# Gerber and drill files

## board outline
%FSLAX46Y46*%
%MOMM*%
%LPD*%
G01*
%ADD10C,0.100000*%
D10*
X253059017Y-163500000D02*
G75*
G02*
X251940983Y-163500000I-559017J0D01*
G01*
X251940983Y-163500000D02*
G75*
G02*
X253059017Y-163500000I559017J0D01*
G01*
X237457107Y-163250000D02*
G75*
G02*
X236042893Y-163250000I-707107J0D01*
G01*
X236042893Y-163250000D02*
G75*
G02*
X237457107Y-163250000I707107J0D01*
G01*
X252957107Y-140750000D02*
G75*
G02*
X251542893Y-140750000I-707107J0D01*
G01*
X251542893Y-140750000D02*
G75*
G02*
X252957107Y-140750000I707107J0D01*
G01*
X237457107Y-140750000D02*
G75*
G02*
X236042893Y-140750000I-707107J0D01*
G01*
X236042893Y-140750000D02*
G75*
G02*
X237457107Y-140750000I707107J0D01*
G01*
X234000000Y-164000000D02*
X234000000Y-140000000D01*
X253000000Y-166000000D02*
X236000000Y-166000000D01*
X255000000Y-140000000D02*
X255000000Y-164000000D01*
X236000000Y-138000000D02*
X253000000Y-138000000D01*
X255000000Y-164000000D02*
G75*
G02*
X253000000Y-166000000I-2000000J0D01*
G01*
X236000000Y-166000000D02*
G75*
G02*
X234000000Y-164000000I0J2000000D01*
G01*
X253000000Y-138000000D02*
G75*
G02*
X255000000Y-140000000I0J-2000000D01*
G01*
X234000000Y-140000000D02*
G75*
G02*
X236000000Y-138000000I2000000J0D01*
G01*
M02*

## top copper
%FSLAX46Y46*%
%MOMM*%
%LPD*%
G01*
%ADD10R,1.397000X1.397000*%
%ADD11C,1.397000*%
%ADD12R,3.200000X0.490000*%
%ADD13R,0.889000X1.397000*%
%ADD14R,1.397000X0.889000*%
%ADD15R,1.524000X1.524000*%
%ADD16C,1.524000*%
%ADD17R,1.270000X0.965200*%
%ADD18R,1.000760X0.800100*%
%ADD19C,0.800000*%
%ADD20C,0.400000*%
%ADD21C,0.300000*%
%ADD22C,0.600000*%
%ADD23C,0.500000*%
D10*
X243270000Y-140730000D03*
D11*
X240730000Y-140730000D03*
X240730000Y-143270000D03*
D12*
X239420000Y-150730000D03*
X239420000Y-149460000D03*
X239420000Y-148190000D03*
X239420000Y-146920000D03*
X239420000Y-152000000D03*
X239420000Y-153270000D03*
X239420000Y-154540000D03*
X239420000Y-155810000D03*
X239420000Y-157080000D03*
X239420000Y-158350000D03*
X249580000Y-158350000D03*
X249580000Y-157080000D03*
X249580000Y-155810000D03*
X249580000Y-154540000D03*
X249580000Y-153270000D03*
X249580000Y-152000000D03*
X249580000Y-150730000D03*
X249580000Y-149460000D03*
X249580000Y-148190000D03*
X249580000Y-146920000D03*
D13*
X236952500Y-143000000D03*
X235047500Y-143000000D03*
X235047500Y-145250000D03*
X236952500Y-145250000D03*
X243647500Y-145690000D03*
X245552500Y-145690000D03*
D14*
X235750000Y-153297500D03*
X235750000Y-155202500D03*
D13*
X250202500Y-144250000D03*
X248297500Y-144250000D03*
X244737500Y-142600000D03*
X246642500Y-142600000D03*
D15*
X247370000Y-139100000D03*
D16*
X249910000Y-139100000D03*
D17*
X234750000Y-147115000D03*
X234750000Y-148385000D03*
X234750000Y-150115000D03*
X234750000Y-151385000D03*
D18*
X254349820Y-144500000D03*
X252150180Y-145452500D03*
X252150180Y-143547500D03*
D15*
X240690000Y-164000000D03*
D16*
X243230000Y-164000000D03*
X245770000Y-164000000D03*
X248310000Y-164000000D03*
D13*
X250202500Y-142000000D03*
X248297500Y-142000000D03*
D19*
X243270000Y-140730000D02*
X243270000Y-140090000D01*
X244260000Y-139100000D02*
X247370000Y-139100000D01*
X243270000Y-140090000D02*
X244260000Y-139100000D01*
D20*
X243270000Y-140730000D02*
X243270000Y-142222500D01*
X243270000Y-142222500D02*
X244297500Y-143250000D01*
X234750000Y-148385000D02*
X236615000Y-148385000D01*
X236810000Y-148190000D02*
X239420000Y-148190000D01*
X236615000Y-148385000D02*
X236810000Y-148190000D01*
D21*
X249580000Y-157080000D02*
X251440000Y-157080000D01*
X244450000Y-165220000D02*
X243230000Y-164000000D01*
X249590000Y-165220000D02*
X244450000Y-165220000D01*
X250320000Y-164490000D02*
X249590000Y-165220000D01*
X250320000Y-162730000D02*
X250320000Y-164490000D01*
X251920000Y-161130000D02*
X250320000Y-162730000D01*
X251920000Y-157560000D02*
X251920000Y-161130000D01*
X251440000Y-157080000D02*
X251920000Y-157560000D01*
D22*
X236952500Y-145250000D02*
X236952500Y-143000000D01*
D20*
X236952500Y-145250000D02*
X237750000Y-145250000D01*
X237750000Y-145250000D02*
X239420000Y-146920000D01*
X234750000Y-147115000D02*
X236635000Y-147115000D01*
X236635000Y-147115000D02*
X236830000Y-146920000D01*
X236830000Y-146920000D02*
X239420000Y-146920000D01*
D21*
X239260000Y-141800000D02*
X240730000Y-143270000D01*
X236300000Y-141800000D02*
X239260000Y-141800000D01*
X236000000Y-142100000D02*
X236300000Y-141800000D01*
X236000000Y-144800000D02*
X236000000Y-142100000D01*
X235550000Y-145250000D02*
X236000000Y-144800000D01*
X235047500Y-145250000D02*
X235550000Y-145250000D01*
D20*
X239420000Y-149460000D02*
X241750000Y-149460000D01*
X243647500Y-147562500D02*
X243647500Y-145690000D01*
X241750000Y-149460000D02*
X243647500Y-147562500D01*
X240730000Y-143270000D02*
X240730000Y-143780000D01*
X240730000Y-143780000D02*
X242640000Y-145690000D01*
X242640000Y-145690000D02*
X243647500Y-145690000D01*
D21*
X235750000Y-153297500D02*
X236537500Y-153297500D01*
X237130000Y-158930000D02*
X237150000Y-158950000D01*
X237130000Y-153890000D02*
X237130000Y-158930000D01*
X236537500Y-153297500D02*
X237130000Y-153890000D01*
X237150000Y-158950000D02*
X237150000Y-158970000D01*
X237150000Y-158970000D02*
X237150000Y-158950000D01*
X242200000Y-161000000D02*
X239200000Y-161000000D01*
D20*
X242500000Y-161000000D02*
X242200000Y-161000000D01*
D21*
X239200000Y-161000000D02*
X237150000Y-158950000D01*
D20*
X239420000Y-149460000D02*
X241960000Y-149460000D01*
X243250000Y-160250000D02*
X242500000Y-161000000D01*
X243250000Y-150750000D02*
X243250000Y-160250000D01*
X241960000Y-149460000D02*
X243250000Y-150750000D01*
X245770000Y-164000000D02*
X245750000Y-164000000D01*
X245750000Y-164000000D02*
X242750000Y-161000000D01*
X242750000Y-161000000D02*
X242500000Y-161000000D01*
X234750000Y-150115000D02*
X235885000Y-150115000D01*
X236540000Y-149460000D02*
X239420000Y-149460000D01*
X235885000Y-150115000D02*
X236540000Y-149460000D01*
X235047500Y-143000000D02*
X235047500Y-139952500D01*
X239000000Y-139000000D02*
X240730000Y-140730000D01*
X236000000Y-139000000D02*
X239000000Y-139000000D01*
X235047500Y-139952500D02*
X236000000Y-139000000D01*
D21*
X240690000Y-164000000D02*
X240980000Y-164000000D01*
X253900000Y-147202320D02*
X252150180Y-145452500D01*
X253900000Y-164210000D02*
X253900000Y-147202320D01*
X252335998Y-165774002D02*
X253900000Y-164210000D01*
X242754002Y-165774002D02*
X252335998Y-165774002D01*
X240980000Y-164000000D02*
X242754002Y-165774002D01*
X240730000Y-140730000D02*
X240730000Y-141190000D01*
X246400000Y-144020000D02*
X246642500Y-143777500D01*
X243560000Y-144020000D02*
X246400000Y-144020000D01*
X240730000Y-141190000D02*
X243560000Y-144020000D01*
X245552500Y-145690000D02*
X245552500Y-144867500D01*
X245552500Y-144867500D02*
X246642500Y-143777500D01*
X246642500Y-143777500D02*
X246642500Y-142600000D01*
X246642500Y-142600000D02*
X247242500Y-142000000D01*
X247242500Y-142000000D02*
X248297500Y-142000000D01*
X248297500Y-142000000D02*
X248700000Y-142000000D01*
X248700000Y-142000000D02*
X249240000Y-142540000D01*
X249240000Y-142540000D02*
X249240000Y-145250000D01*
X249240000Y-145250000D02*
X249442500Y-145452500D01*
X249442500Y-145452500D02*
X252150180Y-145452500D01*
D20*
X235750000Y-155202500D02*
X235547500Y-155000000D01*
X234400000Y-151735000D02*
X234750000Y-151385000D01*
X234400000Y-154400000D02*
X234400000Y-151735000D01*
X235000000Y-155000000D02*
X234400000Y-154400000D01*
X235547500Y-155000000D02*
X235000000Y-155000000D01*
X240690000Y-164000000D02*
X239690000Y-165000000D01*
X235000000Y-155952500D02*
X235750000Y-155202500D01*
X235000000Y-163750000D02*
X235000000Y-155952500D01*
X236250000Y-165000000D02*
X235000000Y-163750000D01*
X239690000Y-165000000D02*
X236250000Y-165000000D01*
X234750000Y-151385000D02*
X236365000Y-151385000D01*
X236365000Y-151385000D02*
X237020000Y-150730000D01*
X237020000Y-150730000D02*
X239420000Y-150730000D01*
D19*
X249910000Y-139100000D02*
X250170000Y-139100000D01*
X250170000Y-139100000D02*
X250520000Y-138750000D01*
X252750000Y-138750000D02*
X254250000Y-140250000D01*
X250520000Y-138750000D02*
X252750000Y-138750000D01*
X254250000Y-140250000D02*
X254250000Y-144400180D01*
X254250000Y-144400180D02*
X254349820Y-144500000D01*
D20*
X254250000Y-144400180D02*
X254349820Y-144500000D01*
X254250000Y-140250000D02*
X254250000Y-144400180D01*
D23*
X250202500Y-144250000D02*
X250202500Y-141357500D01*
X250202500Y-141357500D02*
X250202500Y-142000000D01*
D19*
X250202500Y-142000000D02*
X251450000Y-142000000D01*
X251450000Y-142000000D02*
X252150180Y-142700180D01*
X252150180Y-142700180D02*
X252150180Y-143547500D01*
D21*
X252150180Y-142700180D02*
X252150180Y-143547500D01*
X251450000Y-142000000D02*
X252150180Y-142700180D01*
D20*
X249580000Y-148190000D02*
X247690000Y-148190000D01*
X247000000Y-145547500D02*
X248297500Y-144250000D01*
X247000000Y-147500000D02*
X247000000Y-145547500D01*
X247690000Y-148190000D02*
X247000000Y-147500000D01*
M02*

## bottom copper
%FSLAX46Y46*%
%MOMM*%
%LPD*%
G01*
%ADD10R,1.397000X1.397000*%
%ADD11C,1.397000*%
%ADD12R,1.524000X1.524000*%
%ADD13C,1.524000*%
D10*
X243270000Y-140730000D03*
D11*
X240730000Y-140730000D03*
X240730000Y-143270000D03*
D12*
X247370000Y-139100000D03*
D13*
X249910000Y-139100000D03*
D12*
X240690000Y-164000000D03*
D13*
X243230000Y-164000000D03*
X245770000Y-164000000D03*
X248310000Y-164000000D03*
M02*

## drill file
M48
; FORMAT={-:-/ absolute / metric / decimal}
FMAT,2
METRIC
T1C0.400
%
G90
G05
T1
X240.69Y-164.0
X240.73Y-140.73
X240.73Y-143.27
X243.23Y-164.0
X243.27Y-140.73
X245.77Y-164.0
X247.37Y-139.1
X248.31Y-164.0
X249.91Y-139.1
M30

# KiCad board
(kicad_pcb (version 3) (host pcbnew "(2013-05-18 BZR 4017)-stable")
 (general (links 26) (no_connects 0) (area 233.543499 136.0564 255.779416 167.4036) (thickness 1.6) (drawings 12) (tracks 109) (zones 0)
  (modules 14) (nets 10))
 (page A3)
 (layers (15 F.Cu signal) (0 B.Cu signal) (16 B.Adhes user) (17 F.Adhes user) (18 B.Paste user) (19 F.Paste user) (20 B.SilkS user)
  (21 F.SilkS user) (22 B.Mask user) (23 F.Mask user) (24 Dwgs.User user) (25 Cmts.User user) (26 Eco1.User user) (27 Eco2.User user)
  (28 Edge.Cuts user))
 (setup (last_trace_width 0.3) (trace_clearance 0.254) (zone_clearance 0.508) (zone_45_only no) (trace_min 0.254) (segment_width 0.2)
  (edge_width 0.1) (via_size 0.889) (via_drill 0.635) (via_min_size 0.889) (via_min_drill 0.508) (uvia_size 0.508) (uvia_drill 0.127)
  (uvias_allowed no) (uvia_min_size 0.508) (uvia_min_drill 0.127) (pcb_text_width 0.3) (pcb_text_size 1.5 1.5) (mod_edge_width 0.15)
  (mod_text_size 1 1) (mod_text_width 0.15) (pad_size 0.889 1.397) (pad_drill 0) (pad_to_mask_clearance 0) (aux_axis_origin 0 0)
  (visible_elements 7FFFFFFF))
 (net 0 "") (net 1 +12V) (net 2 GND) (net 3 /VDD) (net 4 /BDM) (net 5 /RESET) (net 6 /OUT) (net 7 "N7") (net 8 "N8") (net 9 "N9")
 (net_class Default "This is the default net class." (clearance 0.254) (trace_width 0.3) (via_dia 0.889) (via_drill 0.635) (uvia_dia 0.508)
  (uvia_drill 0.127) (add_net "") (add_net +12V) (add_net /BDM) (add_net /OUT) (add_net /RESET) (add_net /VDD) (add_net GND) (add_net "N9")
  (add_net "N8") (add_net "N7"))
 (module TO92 (layer F.Cu) (at 242 142)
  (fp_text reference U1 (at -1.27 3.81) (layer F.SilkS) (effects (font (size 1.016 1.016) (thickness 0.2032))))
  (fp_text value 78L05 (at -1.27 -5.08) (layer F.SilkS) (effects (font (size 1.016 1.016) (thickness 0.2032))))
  (pad 1 thru_hole rect (at 1.27 -1.27) (size 1.397 1.397) (drill 0.4) (layers *.Cu *.Mask F.SilkS) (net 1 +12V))
  (pad 2 thru_hole circle (at -1.27 -1.27) (size 1.397 1.397) (drill 0.4) (layers *.Cu *.Mask F.SilkS) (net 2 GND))
  (pad 3 thru_hole circle (at -1.27 1.27) (size 1.397 1.397) (drill 0.4) (layers *.Cu *.Mask F.SilkS) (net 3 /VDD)))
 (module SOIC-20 (layer F.Cu) (at 244.5 152)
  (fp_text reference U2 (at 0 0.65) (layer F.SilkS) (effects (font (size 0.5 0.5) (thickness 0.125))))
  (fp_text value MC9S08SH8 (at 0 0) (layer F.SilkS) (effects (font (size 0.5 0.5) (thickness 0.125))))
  (pad 4 smd rect (at -5.08 -1.27) (size 3.2 0.49) (layers F.Cu F.Paste F.Mask) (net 2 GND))
  (pad 3 smd rect (at -5.08 -2.54) (size 3.2 0.49) (layers F.Cu F.Paste F.Mask) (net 3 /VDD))
  (pad 2 smd rect (at -5.08 -3.81) (size 3.2 0.49) (layers F.Cu F.Paste F.Mask) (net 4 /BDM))
  (pad 1 smd rect (at -5.08 -5.08) (size 3.2 0.49) (layers F.Cu F.Paste F.Mask) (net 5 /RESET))
  (pad 5 smd rect (at -5.08 0) (size 3.2 0.49) (layers F.Cu F.Paste F.Mask))
  (pad 6 smd rect (at -5.08 1.27) (size 3.2 0.49) (layers F.Cu F.Paste F.Mask))
  (pad 7 smd rect (at -5.08 2.54) (size 3.2 0.49) (layers F.Cu F.Paste F.Mask))
  (pad 8 smd rect (at -5.08 3.81) (size 3.2 0.49) (layers F.Cu F.Paste F.Mask))
  (pad 9 smd rect (at -5.08 5.08) (size 3.2 0.49) (layers F.Cu F.Paste F.Mask))
  (pad 10 smd rect (at -5.08 6.35) (size 3.2 0.49) (layers F.Cu F.Paste F.Mask))
  (pad 11 smd rect (at 5.08 6.35) (size 3.2 0.49) (layers F.Cu F.Paste F.Mask))
  (pad 12 smd rect (at 5.08 5.08) (size 3.2 0.49) (layers F.Cu F.Paste F.Mask) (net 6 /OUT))
  (pad 13 smd rect (at 5.08 3.81) (size 3.2 0.49) (layers F.Cu F.Paste F.Mask))
  (pad 14 smd rect (at 5.08 2.54) (size 3.2 0.49) (layers F.Cu F.Paste F.Mask))
  (pad 15 smd rect (at 5.08 1.27) (size 3.2 0.49) (layers F.Cu F.Paste F.Mask))
  (pad 16 smd rect (at 5.08 0) (size 3.2 0.49) (layers F.Cu F.Paste F.Mask))
  (pad 17 smd rect (at 5.08 -1.27) (size 3.2 0.49) (layers F.Cu F.Paste F.Mask))
  (pad 18 smd rect (at 5.08 -2.54) (size 3.2 0.49) (layers F.Cu F.Paste F.Mask))
  (pad 19 smd rect (at 5.08 -3.81) (size 3.2 0.49) (layers F.Cu F.Paste F.Mask) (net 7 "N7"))
  (pad 20 smd rect (at 5.08 -5.08) (size 3.2 0.49) (layers F.Cu F.Paste F.Mask)))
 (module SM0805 (layer F.Cu) (at 236 143 180)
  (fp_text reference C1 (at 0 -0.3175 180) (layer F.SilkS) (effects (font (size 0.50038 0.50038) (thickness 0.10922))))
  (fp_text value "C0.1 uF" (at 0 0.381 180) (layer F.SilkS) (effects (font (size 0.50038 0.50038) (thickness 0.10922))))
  (pad 1 smd rect (at -0.9525 0 180) (size 0.889 1.397) (layers F.Cu F.Paste F.Mask) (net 5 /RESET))
  (pad 2 smd rect (at 0.9525 0 180) (size 0.889 1.397) (layers F.Cu F.Paste F.Mask) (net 2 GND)))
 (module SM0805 (layer F.Cu) (at 236 145.25)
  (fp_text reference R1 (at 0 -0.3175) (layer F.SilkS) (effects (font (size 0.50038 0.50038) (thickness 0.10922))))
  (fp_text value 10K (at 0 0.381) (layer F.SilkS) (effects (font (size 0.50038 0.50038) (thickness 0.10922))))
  (pad 1 smd rect (at -0.9525 0) (size 0.889 1.397) (layers F.Cu F.Paste F.Mask) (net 3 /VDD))
  (pad 2 smd rect (at 0.9525 0) (size 0.889 1.397) (layers F.Cu F.Paste F.Mask) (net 5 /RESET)))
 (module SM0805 (layer F.Cu) (at 244.6 145.69)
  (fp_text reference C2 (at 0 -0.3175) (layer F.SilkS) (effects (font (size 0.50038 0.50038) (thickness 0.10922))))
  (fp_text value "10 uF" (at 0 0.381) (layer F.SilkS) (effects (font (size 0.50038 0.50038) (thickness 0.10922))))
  (pad 1 smd rect (at -0.9525 0) (size 0.889 1.397) (layers F.Cu F.Paste F.Mask) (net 3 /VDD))
  (pad 2 smd rect (at 0.9525 0) (size 0.889 1.397) (layers F.Cu F.Paste F.Mask) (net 2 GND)))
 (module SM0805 (layer F.Cu) (at 235.75 154.25 270)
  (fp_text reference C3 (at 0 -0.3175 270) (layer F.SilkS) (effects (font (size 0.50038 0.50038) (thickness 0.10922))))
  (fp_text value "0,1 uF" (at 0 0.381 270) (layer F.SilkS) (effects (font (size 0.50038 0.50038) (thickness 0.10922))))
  (pad 1 smd rect (at -0.9525 0 270) (size 0.889 1.397) (layers F.Cu F.Paste F.Mask) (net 3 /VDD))
  (pad 2 smd rect (at 0.9525 0 270) (size 0.889 1.397) (layers F.Cu F.Paste F.Mask) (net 2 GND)))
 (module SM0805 (layer F.Cu) (at 249.25 144.25 180)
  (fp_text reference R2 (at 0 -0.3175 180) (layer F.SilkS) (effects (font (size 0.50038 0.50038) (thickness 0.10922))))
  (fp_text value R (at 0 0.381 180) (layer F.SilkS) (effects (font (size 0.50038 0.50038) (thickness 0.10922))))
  (pad 1 smd rect (at -0.9525 0 180) (size 0.889 1.397) (layers F.Cu F.Paste F.Mask) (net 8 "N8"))
  (pad 2 smd rect (at 0.9525 0 180) (size 0.889 1.397) (layers F.Cu F.Paste F.Mask) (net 7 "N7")))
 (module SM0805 (layer F.Cu) (at 245.69 142.6)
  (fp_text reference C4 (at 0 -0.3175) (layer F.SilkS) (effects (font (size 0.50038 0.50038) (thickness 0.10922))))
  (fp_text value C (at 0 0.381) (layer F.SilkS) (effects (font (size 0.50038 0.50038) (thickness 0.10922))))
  (pad 1 smd rect (at -0.9525 0) (size 0.889 1.397) (layers F.Cu F.Paste F.Mask) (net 1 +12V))
  (pad 2 smd rect (at 0.9525 0) (size 0.889 1.397) (layers F.Cu F.Paste F.Mask) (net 2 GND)))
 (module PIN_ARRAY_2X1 (layer F.Cu) (at 248.64 139.1)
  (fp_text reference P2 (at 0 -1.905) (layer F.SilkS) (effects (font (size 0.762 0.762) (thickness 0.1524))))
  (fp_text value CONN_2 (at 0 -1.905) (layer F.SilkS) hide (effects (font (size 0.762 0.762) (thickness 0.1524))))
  (pad 1 thru_hole rect (at -1.27 0) (size 1.524 1.524) (drill 0.4) (layers *.Cu *.Mask F.SilkS) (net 1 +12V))
  (pad 2 thru_hole circle (at 1.27 0) (size 1.524 1.524) (drill 0.4) (layers *.Cu *.Mask F.SilkS) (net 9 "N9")))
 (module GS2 (layer F.Cu) (at 234.75 147.75)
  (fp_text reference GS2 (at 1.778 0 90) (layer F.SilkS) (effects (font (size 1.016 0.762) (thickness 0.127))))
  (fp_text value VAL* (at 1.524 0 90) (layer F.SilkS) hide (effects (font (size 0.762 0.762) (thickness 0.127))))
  (pad 1 smd rect (at 0 -0.635) (size 1.27 0.9652) (layers F.Cu F.Paste F.Mask) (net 5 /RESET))
  (pad 2 smd rect (at 0 0.635) (size 1.27 0.9652) (layers F.Cu F.Paste F.Mask) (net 4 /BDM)))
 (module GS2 (layer F.Cu) (at 234.75 150.75)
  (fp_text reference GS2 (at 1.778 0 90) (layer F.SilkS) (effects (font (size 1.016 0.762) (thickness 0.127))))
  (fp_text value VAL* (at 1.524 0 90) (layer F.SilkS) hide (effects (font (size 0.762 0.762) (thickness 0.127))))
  (pad 1 smd rect (at 0 -0.635) (size 1.27 0.9652) (layers F.Cu F.Paste F.Mask) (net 3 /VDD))
  (pad 2 smd rect (at 0 0.635) (size 1.27 0.9652) (layers F.Cu F.Paste F.Mask) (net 2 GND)))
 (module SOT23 (layer F.Cu) (at 253.25 144.5 270)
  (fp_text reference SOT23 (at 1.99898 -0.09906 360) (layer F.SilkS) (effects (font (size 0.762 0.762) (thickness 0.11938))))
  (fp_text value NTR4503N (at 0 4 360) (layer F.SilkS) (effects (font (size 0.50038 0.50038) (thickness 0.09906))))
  (pad 3 smd rect (at 0 -1.09982 270) (size 0.8001 1.00076) (layers F.Cu F.Paste F.Mask) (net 9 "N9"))
  (pad 2 smd rect (at 0.9525 1.09982 270) (size 0.8001 1.00076) (layers F.Cu F.Paste F.Mask) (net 2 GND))
  (pad 1 smd rect (at -0.9525 1.09982 270) (size 0.8001 1.00076) (layers F.Cu F.Paste F.Mask) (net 8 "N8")))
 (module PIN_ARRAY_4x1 (layer F.Cu) (at 244.5 164)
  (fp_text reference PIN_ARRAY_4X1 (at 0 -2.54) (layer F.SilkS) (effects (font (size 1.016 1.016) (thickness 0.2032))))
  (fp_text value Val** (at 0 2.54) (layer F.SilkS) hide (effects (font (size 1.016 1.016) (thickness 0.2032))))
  (pad 1 thru_hole rect (at -3.81 0) (size 1.524 1.524) (drill 0.4) (layers *.Cu *.Mask F.SilkS) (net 2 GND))
  (pad 2 thru_hole circle (at -1.27 0) (size 1.524 1.524) (drill 0.4) (layers *.Cu *.Mask F.SilkS) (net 6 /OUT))
  (pad 3 thru_hole circle (at 1.27 0) (size 1.524 1.524) (drill 0.4) (layers *.Cu *.Mask F.SilkS) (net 3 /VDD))
  (pad 4 thru_hole circle (at 3.81 0) (size 1.524 1.524) (drill 0.4) (layers *.Cu *.Mask F.SilkS)))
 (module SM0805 (layer F.Cu) (at 249.25 142 180)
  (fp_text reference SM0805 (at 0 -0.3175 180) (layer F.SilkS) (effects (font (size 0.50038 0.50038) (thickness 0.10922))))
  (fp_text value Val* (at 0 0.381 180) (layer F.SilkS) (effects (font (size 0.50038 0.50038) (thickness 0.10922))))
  (pad 1 smd rect (at -0.9525 0 180) (size 0.889 1.397) (layers F.Cu F.Paste F.Mask) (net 8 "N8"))
  (pad 2 smd rect (at 0.9525 0 180) (size 0.889 1.397) (layers F.Cu F.Paste F.Mask) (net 2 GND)))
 (gr_circle (center 252.5 163.5) (end 253 163.75) (layer Edge.Cuts) (width 0.1))
 (gr_circle (center 236.75 163.25) (end 237.25 163.75) (layer Edge.Cuts) (width 0.1))
 (gr_circle (center 252.25 140.75) (end 252.75 140.25) (layer Edge.Cuts) (width 0.1))
 (gr_circle (center 236.75 140.75) (end 236.25 140.25) (layer Edge.Cuts) (width 0.1))
 (gr_line (start 234 164) (end 234 140) (angle 90) (layer Edge.Cuts) (width 0.1))
 (gr_line (start 253 166) (end 236 166) (angle 90) (layer Edge.Cuts) (width 0.1))
 (gr_line (start 255 140) (end 255 164) (angle 90) (layer Edge.Cuts) (width 0.1))
 (gr_line (start 236 138) (end 253 138) (angle 90) (layer Edge.Cuts) (width 0.1))
 (gr_arc (start 253 164) (end 255 164) (angle 90) (layer Edge.Cuts) (width 0.1))
 (gr_arc (start 236 164) (end 236 166) (angle 90) (layer Edge.Cuts) (width 0.1))
 (gr_arc (start 253 140) (end 253 138) (angle 90) (layer Edge.Cuts) (width 0.1))
 (gr_arc (start 236 140) (end 234 140) (angle 90) (layer Edge.Cuts) (width 0.1))
 (segment (start 243.27 140.73) (end 243.27 140.09) (width 0.8) (layer F.Cu) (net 1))
 (segment (start 244.26 139.1) (end 247.37 139.1) (width 0.8) (layer F.Cu) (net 1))
 (segment (start 243.27 140.09) (end 244.26 139.1) (width 0.8) (layer F.Cu) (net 1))
 (segment (start 243.27 140.73) (end 243.27 142.2225) (width 0.4) (layer F.Cu) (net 1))
 (segment (start 243.27 142.2225) (end 244.2975 143.25) (width 0.4) (layer F.Cu) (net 1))
 (segment (start 234.75 148.385) (end 236.615 148.385) (width 0.4) (layer F.Cu) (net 4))
 (segment (start 236.81 148.19) (end 239.42 148.19) (width 0.4) (layer F.Cu) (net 4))
 (segment (start 236.615 148.385) (end 236.81 148.19) (width 0.4) (layer F.Cu) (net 4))
 (segment (start 249.58 157.08) (end 251.44 157.08) (width 0.3) (layer F.Cu) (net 6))
 (segment (start 244.45 165.22) (end 243.23 164) (width 0.3) (layer F.Cu) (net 6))
 (segment (start 249.59 165.22) (end 244.45 165.22) (width 0.3) (layer F.Cu) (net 6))
 (segment (start 250.32 164.49) (end 249.59 165.22) (width 0.3) (layer F.Cu) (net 6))
 (segment (start 250.32 162.73) (end 250.32 164.49) (width 0.3) (layer F.Cu) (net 6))
 (segment (start 251.92 161.13) (end 250.32 162.73) (width 0.3) (layer F.Cu) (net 6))
 (segment (start 251.92 157.56) (end 251.92 161.13) (width 0.3) (layer F.Cu) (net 6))
 (segment (start 251.44 157.08) (end 251.92 157.56) (width 0.3) (layer F.Cu) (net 6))
 (segment (start 236.9525 145.25) (end 236.9525 143) (width 0.6) (layer F.Cu) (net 5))
 (segment (start 236.9525 145.25) (end 237.75 145.25) (width 0.4) (layer F.Cu) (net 5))
 (segment (start 237.75 145.25) (end 239.42 146.92) (width 0.4) (layer F.Cu) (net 5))
 (segment (start 234.75 147.115) (end 236.635 147.115) (width 0.4) (layer F.Cu) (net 5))
 (segment (start 236.635 147.115) (end 236.83 146.92) (width 0.4) (layer F.Cu) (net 5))
 (segment (start 236.83 146.92) (end 239.42 146.92) (width 0.4) (layer F.Cu) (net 5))
 (segment (start 239.26 141.8) (end 240.73 143.27) (width 0.3) (layer F.Cu) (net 3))
 (segment (start 236.3 141.8) (end 239.26 141.8) (width 0.3) (layer F.Cu) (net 3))
 (segment (start 236 142.1) (end 236.3 141.8) (width 0.3) (layer F.Cu) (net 3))
 (segment (start 236 144.8) (end 236 142.1) (width 0.3) (layer F.Cu) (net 3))
 (segment (start 235.55 145.25) (end 236 144.8) (width 0.3) (layer F.Cu) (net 3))
 (segment (start 235.0475 145.25) (end 235.55 145.25) (width 0.3) (layer F.Cu) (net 3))
 (segment (start 239.42 149.46) (end 241.75 149.46) (width 0.4) (layer F.Cu) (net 3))
 (segment (start 243.6475 147.5625) (end 243.6475 145.69) (width 0.4) (layer F.Cu) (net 3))
 (segment (start 241.75 149.46) (end 243.6475 147.5625) (width 0.4) (layer F.Cu) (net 3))
 (segment (start 240.73 143.27) (end 240.73 143.78) (width 0.4) (layer F.Cu) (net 3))
 (segment (start 240.73 143.78) (end 242.64 145.69) (width 0.4) (layer F.Cu) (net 3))
 (segment (start 242.64 145.69) (end 243.6475 145.69) (width 0.4) (layer F.Cu) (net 3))
 (segment (start 235.75 153.2975) (end 236.5375 153.2975) (width 0.3) (layer F.Cu) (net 3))
 (segment (start 237.13 158.93) (end 237.15 158.95) (width 0.3) (layer F.Cu) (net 3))
 (segment (start 237.13 153.89) (end 237.13 158.93) (width 0.3) (layer F.Cu) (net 3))
 (segment (start 236.5375 153.2975) (end 237.13 153.89) (width 0.3) (layer F.Cu) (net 3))
 (segment (start 237.15 158.95) (end 237.15 158.97) (width 0.3) (layer F.Cu) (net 3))
 (segment (start 237.15 158.97) (end 237.15 158.95) (width 0.3) (layer F.Cu) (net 3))
 (segment (start 242.2 161) (end 239.2 161) (width 0.3) (layer F.Cu) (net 3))
 (segment (start 242.5 161) (end 242.2 161) (width 0.4) (layer F.Cu) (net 3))
 (segment (start 239.2 161) (end 237.15 158.95) (width 0.3) (layer F.Cu) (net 3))
 (segment (start 239.42 149.46) (end 241.96 149.46) (width 0.4) (layer F.Cu) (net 3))
 (segment (start 243.25 160.25) (end 242.5 161) (width 0.4) (layer F.Cu) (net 3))
 (segment (start 243.25 150.75) (end 243.25 160.25) (width 0.4) (layer F.Cu) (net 3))
 (segment (start 241.96 149.46) (end 243.25 150.75) (width 0.4) (layer F.Cu) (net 3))
 (segment (start 245.77 164) (end 245.75 164) (width 0.4) (layer F.Cu) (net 3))
 (segment (start 245.75 164) (end 242.75 161) (width 0.4) (layer F.Cu) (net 3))
 (segment (start 242.75 161) (end 242.5 161) (width 0.4) (layer F.Cu) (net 3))
 (segment (start 234.75 150.115) (end 235.885 150.115) (width 0.4) (layer F.Cu) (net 3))
 (segment (start 236.54 149.46) (end 239.42 149.46) (width 0.4) (layer F.Cu) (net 3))
 (segment (start 235.885 150.115) (end 236.54 149.46) (width 0.4) (layer F.Cu) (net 3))
 (segment (start 235.0475 143) (end 235.0475 139.9525) (width 0.4) (layer F.Cu) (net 2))
 (segment (start 239 139) (end 240.73 140.73) (width 0.4) (layer F.Cu) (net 2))
 (segment (start 236 139) (end 239 139) (width 0.4) (layer F.Cu) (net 2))
 (segment (start 235.0475 139.9525) (end 236 139) (width 0.4) (layer F.Cu) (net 2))
 (segment (start 240.69 164) (end 240.98 164) (width 0.3) (layer F.Cu) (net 2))
 (segment (start 253.9 147.20232) (end 252.15018 145.4525) (width 0.3) (layer F.Cu) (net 2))
 (segment (start 253.9 164.21) (end 253.9 147.20232) (width 0.3) (layer F.Cu) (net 2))
 (segment (start 252.335998 165.774002) (end 253.9 164.21) (width 0.3) (layer F.Cu) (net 2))
 (segment (start 242.754002 165.774002) (end 252.335998 165.774002) (width 0.3) (layer F.Cu) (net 2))
 (segment (start 240.98 164) (end 242.754002 165.774002) (width 0.3) (layer F.Cu) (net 2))
 (segment (start 240.73 140.73) (end 240.73 141.19) (width 0.3) (layer F.Cu) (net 2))
 (segment (start 246.4 144.02) (end 246.6425 143.7775) (width 0.3) (layer F.Cu) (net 2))
 (segment (start 243.56 144.02) (end 246.4 144.02) (width 0.3) (layer F.Cu) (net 2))
 (segment (start 240.73 141.19) (end 243.56 144.02) (width 0.3) (layer F.Cu) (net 2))
 (segment (start 245.5525 145.69) (end 245.5525 144.8675) (width 0.3) (layer F.Cu) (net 2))
 (segment (start 245.5525 144.8675) (end 246.6425 143.7775) (width 0.3) (layer F.Cu) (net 2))
 (segment (start 246.6425 143.7775) (end 246.6425 142.6) (width 0.3) (layer F.Cu) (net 2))
 (segment (start 246.6425 142.6) (end 247.2425 142) (width 0.3) (layer F.Cu) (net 2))
 (segment (start 247.2425 142) (end 248.2975 142) (width 0.3) (layer F.Cu) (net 2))
 (segment (start 248.2975 142) (end 248.7 142) (width 0.3) (layer F.Cu) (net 2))
 (segment (start 248.7 142) (end 249.24 142.54) (width 0.3) (layer F.Cu) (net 2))
 (segment (start 249.24 142.54) (end 249.24 145.25) (width 0.3) (layer F.Cu) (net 2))
 (segment (start 249.24 145.25) (end 249.4425 145.4525) (width 0.3) (layer F.Cu) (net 2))
 (segment (start 249.4425 145.4525) (end 252.15018 145.4525) (width 0.3) (layer F.Cu) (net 2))
 (segment (start 235.75 155.2025) (end 235.5475 155) (width 0.4) (layer F.Cu) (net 2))
 (segment (start 234.4 151.735) (end 234.75 151.385) (width 0.4) (layer F.Cu) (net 2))
 (segment (start 234.4 154.4) (end 234.4 151.735) (width 0.4) (layer F.Cu) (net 2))
 (segment (start 235 155) (end 234.4 154.4) (width 0.4) (layer F.Cu) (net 2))
 (segment (start 235.5475 155) (end 235 155) (width 0.4) (layer F.Cu) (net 2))
 (segment (start 240.69 164) (end 239.69 165) (width 0.4) (layer F.Cu) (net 2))
 (segment (start 235 155.9525) (end 235.75 155.2025) (width 0.4) (layer F.Cu) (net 2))
 (segment (start 235 163.75) (end 235 155.9525) (width 0.4) (layer F.Cu) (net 2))
 (segment (start 236.25 165) (end 235 163.75) (width 0.4) (layer F.Cu) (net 2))
 (segment (start 239.69 165) (end 236.25 165) (width 0.4) (layer F.Cu) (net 2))
 (segment (start 234.75 151.385) (end 236.365 151.385) (width 0.4) (layer F.Cu) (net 2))
 (segment (start 236.365 151.385) (end 237.02 150.73) (width 0.4) (layer F.Cu) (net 2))
 (segment (start 237.02 150.73) (end 239.42 150.73) (width 0.4) (layer F.Cu) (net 2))
 (segment (start 249.91 139.1) (end 250.17 139.1) (width 0.8) (layer F.Cu) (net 9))
 (segment (start 250.17 139.1) (end 250.52 138.75) (width 0.8) (layer F.Cu) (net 9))
 (segment (start 252.75 138.75) (end 254.25 140.25) (width 0.8) (layer F.Cu) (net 9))
 (segment (start 250.52 138.75) (end 252.75 138.75) (width 0.8) (layer F.Cu) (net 9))
 (segment (start 254.25 140.25) (end 254.25 144.40018) (width 0.8) (layer F.Cu) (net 9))
 (segment (start 254.25 144.40018) (end 254.34982 144.5) (width 0.8) (layer F.Cu) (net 9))
 (segment (start 254.25 144.40018) (end 254.34982 144.5) (width 0.4) (layer F.Cu) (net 9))
 (segment (start 254.25 140.25) (end 254.25 144.40018) (width 0.4) (layer F.Cu) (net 9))
 (segment (start 250.2025 144.25) (end 250.2025 141.3575) (width 0.5) (layer F.Cu) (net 8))
 (segment (start 250.2025 141.3575) (end 250.2025 142) (width 0.5) (layer F.Cu) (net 8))
 (segment (start 250.2025 142) (end 251.45 142) (width 0.8) (layer F.Cu) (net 8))
 (segment (start 251.45 142) (end 252.15018 142.70018) (width 0.8) (layer F.Cu) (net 8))
 (segment (start 252.15018 142.70018) (end 252.15018 143.5475) (width 0.8) (layer F.Cu) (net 8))
 (segment (start 252.15018 142.70018) (end 252.15018 143.5475) (width 0.3) (layer F.Cu) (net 8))
 (segment (start 251.45 142) (end 252.15018 142.70018) (width 0.3) (layer F.Cu) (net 8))
 (segment (start 249.58 148.19) (end 247.69 148.19) (width 0.4) (layer F.Cu) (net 7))
 (segment (start 247 145.5475) (end 248.2975 144.25) (width 0.4) (layer F.Cu) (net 7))
 (segment (start 247 147.5) (end 247 145.5475) (width 0.4) (layer F.Cu) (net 7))
 (segment (start 247.69 148.19) (end 247 147.5) (width 0.4) (layer F.Cu) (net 7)))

